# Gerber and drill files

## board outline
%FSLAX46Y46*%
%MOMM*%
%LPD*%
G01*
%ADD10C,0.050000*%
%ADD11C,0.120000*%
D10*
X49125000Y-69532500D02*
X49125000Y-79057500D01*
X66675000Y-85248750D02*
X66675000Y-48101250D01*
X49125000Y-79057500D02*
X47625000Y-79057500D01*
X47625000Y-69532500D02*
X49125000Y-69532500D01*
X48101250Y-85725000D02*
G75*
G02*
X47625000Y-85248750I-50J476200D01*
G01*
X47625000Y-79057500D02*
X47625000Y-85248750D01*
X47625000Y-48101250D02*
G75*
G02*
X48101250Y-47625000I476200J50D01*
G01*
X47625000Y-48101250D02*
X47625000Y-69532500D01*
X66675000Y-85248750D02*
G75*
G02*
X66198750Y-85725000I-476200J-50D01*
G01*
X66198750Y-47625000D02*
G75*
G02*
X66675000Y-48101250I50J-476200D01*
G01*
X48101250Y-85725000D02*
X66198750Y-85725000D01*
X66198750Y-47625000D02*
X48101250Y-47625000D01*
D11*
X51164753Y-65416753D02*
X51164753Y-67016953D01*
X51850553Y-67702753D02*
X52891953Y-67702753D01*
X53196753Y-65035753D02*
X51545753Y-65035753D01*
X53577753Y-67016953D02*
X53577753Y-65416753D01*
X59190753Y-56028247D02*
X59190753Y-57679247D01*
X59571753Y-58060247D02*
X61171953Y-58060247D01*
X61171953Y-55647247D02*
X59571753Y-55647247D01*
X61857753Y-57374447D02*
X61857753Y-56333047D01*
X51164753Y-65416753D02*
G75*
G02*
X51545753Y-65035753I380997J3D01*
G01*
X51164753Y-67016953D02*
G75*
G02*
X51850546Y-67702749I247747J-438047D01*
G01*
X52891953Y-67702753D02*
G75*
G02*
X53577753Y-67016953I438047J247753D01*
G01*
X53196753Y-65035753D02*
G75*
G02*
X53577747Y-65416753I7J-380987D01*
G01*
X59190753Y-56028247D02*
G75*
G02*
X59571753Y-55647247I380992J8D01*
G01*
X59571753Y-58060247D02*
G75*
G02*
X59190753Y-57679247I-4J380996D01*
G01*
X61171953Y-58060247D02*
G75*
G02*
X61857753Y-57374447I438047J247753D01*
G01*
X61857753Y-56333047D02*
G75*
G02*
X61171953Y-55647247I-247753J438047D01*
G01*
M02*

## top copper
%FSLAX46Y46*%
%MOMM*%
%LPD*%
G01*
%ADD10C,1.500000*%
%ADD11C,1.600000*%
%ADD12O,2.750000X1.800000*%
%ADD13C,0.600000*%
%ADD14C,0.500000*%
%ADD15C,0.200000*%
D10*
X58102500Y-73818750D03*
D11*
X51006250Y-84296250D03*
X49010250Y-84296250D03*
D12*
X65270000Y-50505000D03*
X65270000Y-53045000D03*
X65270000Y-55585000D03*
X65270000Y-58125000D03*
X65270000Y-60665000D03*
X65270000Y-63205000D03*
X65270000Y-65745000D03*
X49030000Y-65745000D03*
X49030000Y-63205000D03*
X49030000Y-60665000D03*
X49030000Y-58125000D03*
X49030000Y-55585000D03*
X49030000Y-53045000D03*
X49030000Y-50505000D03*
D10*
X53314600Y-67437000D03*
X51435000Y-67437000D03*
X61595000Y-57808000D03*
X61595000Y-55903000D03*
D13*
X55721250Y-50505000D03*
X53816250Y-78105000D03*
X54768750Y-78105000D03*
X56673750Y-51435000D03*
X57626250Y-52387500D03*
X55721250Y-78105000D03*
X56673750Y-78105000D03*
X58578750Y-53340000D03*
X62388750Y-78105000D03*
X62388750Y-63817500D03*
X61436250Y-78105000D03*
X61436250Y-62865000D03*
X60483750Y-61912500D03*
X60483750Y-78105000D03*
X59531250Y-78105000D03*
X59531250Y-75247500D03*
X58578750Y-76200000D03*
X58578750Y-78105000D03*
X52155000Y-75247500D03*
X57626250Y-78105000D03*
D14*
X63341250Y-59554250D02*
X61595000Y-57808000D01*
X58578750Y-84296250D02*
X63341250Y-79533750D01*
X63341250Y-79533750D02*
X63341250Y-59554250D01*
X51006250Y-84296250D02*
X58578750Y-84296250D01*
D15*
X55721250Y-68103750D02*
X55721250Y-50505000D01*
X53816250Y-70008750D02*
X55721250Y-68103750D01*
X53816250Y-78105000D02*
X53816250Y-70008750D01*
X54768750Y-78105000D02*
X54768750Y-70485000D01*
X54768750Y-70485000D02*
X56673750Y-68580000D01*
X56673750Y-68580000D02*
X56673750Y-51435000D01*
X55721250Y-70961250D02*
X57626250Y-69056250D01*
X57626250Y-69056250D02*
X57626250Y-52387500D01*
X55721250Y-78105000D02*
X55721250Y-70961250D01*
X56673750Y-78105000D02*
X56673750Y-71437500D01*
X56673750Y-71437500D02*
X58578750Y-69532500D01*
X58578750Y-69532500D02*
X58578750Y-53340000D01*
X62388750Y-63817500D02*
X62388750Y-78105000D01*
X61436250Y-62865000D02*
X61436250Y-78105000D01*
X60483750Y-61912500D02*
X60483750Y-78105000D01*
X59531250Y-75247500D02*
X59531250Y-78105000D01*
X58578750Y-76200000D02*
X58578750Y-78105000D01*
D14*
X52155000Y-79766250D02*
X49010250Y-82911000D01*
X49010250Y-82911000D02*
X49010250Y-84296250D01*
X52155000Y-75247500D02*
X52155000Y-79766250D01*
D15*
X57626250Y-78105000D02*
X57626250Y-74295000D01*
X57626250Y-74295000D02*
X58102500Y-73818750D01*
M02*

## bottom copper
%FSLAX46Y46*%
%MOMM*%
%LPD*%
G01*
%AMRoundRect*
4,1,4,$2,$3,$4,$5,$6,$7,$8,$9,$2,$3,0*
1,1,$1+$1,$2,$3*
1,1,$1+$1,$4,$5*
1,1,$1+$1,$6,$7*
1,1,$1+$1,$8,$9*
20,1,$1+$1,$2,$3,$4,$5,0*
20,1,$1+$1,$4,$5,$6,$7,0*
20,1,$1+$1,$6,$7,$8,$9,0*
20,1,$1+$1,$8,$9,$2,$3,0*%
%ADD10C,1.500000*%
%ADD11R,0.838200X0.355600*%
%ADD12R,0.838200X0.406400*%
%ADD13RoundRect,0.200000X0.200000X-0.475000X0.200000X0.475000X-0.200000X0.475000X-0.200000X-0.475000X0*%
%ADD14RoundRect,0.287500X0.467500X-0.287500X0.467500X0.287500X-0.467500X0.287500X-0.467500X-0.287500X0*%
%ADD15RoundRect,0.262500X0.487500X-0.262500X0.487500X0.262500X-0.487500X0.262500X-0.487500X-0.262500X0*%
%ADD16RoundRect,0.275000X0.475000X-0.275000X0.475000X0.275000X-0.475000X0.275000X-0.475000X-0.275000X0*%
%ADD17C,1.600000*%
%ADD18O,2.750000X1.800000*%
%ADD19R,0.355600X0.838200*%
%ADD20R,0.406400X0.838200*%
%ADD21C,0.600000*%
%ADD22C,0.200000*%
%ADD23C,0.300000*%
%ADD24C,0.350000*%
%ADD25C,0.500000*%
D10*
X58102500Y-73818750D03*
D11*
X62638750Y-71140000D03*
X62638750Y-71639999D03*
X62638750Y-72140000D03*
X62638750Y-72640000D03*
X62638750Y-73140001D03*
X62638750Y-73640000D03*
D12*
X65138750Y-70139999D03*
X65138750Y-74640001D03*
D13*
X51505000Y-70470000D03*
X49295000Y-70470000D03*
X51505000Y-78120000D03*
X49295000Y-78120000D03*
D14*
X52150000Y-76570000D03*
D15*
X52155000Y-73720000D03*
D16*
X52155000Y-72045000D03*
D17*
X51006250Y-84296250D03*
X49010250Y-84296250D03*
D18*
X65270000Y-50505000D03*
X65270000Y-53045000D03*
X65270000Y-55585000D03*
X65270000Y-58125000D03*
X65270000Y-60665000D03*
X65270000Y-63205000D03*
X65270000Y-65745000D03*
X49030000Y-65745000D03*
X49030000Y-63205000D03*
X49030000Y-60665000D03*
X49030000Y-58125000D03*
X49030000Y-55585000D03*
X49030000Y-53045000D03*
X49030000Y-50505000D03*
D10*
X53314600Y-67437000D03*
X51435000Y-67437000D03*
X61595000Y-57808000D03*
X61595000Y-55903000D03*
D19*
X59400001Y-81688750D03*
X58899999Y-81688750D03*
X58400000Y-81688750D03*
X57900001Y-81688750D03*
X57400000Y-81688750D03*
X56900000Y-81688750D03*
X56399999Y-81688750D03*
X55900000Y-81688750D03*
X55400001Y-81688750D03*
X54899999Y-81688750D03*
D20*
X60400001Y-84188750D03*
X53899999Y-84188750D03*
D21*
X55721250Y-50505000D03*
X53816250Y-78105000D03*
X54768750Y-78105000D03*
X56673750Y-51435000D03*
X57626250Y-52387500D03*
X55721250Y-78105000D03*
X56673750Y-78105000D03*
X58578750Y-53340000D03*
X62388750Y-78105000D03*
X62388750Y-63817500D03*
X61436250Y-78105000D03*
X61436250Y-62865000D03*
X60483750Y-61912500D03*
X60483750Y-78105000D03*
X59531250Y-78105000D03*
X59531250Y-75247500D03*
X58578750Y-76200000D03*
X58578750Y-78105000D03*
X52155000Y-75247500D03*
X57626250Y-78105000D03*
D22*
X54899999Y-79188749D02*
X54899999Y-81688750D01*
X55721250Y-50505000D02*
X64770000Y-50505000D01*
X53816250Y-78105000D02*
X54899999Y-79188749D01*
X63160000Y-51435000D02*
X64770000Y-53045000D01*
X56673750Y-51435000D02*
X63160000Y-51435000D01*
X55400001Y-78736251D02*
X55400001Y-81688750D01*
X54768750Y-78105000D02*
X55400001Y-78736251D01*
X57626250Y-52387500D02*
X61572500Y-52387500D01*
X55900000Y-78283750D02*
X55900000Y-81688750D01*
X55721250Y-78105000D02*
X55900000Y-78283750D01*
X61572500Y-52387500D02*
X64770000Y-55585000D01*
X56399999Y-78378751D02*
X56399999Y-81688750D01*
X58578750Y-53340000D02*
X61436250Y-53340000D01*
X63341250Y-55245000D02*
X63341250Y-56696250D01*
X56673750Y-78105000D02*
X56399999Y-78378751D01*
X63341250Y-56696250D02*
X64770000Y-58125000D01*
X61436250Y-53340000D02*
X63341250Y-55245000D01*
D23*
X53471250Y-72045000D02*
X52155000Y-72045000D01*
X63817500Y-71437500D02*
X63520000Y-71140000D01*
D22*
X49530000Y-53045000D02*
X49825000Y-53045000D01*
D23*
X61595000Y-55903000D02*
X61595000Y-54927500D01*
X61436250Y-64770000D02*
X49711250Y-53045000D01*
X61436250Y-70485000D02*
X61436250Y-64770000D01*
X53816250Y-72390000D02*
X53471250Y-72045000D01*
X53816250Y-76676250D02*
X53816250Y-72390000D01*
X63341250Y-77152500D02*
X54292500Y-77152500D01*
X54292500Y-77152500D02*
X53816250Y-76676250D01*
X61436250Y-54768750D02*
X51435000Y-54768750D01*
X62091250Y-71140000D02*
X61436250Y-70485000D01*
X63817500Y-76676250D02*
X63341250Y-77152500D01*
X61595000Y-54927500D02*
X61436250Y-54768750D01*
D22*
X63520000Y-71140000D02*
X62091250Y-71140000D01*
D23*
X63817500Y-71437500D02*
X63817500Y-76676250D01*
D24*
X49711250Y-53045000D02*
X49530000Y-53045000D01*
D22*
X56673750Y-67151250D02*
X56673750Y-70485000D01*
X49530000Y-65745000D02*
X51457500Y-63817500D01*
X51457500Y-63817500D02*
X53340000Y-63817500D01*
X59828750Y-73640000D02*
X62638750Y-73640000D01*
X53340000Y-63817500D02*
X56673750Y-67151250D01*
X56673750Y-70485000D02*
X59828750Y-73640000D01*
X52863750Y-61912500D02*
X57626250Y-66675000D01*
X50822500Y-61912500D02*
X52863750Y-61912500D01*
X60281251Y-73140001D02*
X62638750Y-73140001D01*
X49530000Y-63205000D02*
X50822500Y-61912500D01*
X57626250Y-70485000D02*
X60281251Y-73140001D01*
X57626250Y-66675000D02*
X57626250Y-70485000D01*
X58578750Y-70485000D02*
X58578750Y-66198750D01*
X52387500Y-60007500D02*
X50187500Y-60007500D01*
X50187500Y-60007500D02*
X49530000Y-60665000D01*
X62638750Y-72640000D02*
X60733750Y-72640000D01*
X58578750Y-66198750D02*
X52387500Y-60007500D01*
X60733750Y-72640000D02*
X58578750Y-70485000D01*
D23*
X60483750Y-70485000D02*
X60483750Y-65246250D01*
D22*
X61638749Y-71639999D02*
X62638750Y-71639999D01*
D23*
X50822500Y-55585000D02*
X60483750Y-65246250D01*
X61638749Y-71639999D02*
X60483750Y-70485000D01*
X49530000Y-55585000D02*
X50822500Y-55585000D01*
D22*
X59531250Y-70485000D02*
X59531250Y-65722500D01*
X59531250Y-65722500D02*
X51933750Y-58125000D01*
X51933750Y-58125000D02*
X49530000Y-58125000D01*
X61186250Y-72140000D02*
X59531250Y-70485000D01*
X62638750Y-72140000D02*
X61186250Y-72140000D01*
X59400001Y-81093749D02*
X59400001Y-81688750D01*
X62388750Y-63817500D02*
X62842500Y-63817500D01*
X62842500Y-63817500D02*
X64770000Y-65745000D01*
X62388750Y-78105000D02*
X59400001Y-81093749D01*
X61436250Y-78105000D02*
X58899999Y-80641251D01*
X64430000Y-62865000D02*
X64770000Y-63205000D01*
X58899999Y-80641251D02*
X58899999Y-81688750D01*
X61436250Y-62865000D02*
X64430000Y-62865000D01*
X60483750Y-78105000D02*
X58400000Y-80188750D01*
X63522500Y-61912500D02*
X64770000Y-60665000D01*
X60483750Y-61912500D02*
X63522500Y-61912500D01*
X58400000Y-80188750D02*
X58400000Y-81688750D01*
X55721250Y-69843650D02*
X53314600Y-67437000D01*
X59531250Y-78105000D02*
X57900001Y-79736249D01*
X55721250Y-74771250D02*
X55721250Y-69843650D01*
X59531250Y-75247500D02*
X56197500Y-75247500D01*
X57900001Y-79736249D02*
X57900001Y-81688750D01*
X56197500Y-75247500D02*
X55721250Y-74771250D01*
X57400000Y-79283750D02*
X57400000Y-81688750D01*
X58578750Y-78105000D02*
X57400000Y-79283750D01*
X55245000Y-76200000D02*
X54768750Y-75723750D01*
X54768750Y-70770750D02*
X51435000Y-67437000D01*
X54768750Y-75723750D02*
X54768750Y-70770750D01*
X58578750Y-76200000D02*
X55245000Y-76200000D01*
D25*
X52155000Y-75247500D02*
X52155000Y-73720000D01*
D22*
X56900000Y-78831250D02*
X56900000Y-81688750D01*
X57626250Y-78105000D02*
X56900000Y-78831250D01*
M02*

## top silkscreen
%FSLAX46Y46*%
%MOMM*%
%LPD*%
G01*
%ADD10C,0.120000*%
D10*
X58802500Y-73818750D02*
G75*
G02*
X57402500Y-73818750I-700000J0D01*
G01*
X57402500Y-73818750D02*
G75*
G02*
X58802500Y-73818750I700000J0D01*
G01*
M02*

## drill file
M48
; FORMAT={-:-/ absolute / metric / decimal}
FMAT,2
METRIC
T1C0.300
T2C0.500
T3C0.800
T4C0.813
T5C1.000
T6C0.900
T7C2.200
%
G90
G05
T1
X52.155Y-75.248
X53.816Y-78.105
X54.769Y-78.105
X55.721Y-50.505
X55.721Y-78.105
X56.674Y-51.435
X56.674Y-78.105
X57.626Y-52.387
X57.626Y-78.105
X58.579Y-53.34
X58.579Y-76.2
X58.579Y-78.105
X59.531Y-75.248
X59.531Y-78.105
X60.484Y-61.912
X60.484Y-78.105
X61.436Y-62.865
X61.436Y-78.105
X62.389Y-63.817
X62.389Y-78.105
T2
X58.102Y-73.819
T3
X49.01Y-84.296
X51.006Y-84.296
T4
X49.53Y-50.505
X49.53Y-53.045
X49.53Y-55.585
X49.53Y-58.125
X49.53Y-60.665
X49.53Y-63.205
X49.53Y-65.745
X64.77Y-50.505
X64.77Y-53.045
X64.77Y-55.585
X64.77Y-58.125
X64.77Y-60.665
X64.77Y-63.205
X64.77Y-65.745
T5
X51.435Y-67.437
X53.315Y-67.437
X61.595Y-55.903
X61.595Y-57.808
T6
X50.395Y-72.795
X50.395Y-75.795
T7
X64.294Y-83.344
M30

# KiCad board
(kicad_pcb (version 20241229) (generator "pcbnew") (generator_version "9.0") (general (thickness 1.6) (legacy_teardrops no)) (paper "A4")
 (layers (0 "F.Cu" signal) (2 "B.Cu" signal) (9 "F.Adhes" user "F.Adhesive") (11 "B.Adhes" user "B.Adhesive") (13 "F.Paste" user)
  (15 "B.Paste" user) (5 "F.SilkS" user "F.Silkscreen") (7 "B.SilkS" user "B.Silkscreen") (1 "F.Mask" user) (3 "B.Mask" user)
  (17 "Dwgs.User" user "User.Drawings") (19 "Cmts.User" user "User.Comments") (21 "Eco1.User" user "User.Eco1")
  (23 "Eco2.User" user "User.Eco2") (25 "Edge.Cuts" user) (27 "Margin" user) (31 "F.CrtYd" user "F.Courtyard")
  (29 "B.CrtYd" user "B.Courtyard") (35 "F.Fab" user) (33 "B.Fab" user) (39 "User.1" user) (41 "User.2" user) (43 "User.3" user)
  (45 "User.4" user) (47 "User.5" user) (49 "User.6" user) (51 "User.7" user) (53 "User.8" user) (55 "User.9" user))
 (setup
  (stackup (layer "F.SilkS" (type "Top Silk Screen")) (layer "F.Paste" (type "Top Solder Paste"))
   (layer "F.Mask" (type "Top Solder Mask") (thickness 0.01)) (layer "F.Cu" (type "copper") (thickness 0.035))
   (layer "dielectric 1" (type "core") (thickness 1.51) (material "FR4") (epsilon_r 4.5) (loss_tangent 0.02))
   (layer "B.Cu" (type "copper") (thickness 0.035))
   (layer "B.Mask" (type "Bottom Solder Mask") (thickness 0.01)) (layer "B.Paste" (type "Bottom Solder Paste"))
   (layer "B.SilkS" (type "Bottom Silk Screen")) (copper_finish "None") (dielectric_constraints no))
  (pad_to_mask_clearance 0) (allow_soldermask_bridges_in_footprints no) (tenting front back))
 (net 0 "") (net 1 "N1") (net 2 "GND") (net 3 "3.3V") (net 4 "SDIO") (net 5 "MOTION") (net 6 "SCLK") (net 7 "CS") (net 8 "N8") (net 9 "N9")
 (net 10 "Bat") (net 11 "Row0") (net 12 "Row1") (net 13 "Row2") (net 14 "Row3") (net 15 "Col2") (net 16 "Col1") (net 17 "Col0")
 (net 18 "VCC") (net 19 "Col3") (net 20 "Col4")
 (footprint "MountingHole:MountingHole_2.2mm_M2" (layer "F.Cu") (at 64.29375 83.34375)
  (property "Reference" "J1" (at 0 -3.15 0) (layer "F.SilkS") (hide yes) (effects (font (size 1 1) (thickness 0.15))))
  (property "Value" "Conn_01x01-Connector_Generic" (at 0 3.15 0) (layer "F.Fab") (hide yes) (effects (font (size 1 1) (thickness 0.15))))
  (pad "" np_thru_hole circle (at 0 0) (size 2.2 2.2) (drill 2.2) (layers "*.Cu" "*.Mask")))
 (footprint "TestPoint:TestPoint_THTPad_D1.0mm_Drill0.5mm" (layer "F.Cu") (at 58.1025 73.81875)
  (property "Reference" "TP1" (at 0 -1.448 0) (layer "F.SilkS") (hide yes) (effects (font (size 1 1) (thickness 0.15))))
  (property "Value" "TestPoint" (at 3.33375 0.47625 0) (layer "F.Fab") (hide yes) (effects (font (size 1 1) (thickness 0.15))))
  (fp_circle (center 0 0) (end 0 0.7) (stroke (width 0.12) (type solid)) (fill no) (layer "F.SilkS"))
  (pad "1" thru_hole circle (at 0 0) (size 1.5 1.5) (drill 0.5) (layers "*.Cu" "*.Mask") (remove_unused_layers no) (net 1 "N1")))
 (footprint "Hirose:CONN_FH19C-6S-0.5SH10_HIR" (layer "B.Cu") (at 64.29375 72.39 -90)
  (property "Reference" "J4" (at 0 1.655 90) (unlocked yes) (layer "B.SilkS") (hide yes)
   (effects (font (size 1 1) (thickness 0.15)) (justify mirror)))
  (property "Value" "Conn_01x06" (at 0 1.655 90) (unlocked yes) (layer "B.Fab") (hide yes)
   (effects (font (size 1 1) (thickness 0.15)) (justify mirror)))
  (pad "1" smd rect (at -1.25 1.655 270) (size 0.3556 0.8382) (layers "B.Cu" "B.Mask" "B.Paste") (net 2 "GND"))
  (pad "2" smd rect (at -0.750001 1.655 270) (size 0.3556 0.8382) (layers "B.Cu" "B.Mask" "B.Paste") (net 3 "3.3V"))
  (pad "3" smd rect (at -0.25 1.655 270) (size 0.3556 0.8382) (layers "B.Cu" "B.Mask" "B.Paste") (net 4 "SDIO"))
  (pad "4" smd rect (at 0.25 1.655 270) (size 0.3556 0.8382) (layers "B.Cu" "B.Mask" "B.Paste") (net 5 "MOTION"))
  (pad "5" smd rect (at 0.750001 1.655 270) (size 0.3556 0.8382) (layers "B.Cu" "B.Mask" "B.Paste") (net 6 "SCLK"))
  (pad "6" smd rect (at 1.25 1.655 270) (size 0.3556 0.8382) (layers "B.Cu" "B.Mask" "B.Paste") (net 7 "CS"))
  (pad "7" smd rect (at -2.250001 -0.845 270) (size 0.4064 0.8382) (layers "B.Cu" "B.Mask" "B.Paste"))
  (pad "8" smd rect (at 2.250001 -0.845 270) (size 0.4064 0.8382) (layers "B.Cu" "B.Mask" "B.Paste")))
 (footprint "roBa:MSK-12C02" (layer "B.Cu") (at 50.395 74.295 -90)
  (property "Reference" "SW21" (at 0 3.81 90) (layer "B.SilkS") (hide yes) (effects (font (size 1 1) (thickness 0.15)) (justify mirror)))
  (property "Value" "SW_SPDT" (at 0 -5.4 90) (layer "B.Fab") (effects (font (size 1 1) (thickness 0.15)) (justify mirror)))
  (pad "" smd roundrect (at -3.825 -1.11 90) (size 1.35 0.8) (layers "B.Cu" "B.Mask" "B.Paste") (roundrect_rratio 0.25))
  (pad "" smd roundrect (at -3.825 1.1 90) (size 1.35 0.8) (layers "B.Cu" "B.Mask" "B.Paste") (roundrect_rratio 0.25))
  (pad "" np_thru_hole circle (at -1.5 0 90) (size 0.9 0.9) (drill 0.9) (layers "*.Cu" "*.Mask"))
  (pad "" np_thru_hole circle (at 1.5 0 90) (size 0.9 0.9) (drill 0.9) (layers "*.Cu" "*.Mask"))
  (pad "" smd roundrect (at 3.825 -1.11 90) (size 1.35 0.8) (layers "B.Cu" "B.Mask" "B.Paste") (roundrect_rratio 0.25))
  (pad "" smd roundrect (at 3.825 1.1 90) (size 1.35 0.8) (layers "B.Cu" "B.Mask" "B.Paste") (roundrect_rratio 0.25))
  (pad "1" smd roundrect (at 2.275 -1.755 90) (size 1.15 1.51) (layers "B.Cu" "B.Mask" "B.Paste") (roundrect_rratio 0.25) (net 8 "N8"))
  (pad "2" smd roundrect (at -0.575 -1.76 90) (size 1.05 1.5) (layers "B.Cu" "B.Mask" "B.Paste") (roundrect_rratio 0.25) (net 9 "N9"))
  (pad "3" smd roundrect (at -2.25 -1.76 90) (size 1.1 1.5) (layers "B.Cu" "B.Mask" "B.Paste") (roundrect_rratio 0.25) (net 2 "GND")))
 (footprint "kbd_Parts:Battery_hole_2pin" (layer "B.Cu") (at 50.00625 84.29625 90)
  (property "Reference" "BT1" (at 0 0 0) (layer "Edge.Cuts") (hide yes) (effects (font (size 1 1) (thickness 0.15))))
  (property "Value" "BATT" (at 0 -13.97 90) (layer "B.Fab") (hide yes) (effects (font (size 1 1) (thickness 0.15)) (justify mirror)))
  (pad "1" thru_hole circle (at 0 1 90) (size 1.6 1.6) (drill 0.8) (layers "*.Cu" "*.Mask" "B.SilkS") (remove_unused_layers no)
   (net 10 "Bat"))
  (pad "2" thru_hole circle (at 0 -0.996 90) (size 1.6 1.6) (drill 0.8) (layers "*.Cu" "*.Mask" "B.SilkS") (remove_unused_layers no)
   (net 9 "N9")))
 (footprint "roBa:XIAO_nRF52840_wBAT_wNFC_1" (layer "B.Cu") (at 57.15 47.625 180)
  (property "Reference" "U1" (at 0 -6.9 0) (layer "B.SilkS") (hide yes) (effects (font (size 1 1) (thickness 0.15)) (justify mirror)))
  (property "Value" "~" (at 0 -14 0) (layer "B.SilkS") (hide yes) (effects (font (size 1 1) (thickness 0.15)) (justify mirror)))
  (fp_line (start 5.985247 -17.791753) (end 5.985247 -19.391953) (stroke (width 0.12) (type solid)) (layer "Edge.Cuts"))
  (fp_line (start 5.299447 -20.077753) (end 4.258047 -20.077753) (stroke (width 0.12) (type solid)) (layer "Edge.Cuts"))
  (fp_line (start 3.953247 -17.410753) (end 5.604247 -17.410753) (stroke (width 0.12) (type solid)) (layer "Edge.Cuts"))
  (fp_line (start 3.572247 -19.391953) (end 3.572247 -17.791753) (stroke (width 0.12) (type solid)) (layer "Edge.Cuts"))
  (fp_line (start -2.040753 -8.403247) (end -2.040753 -10.054247) (stroke (width 0.12) (type solid)) (layer "Edge.Cuts"))
  (fp_line (start -2.421753 -10.435247) (end -4.021953 -10.435247) (stroke (width 0.12) (type solid)) (layer "Edge.Cuts"))
  (fp_line (start -4.021953 -8.022247) (end -2.421753 -8.022247) (stroke (width 0.12) (type solid)) (layer "Edge.Cuts"))
  (fp_line (start -4.707753 -9.749447) (end -4.707753 -8.708047) (stroke (width 0.12) (type solid)) (layer "Edge.Cuts"))
  (fp_arc (start 5.985247 -17.791753) (mid 5.873656 -17.522344) (end 5.604247 -17.410753) (stroke (width 0.12) (type solid))
   (layer "Edge.Cuts"))
  (fp_arc (start 5.985247 -19.391953) (mid 5.381645 -19.474147) (end 5.299447 -20.077753) (stroke (width 0.12) (type solid))
   (layer "Edge.Cuts"))
  (fp_arc (start 4.258047 -20.077753) (mid 4.175856 -19.474144) (end 3.572247 -19.391953) (stroke (width 0.12) (type solid))
   (layer "Edge.Cuts"))
  (fp_arc (start 3.953247 -17.410753) (mid 3.683836 -17.522343) (end 3.572247 -17.791753) (stroke (width 0.12) (type solid))
   (layer "Edge.Cuts"))
  (fp_arc (start -2.040753 -8.403247) (mid -2.152343 -8.133837) (end -2.421753 -8.022247) (stroke (width 0.12) (type solid))
   (layer "Edge.Cuts"))
  (fp_arc (start -2.421753 -10.435247) (mid -2.152344 -10.323656) (end -2.040753 -10.054247) (stroke (width 0.12) (type solid))
   (layer "Edge.Cuts"))
  (fp_arc (start -4.021953 -10.435247) (mid -4.104144 -9.831638) (end -4.707753 -9.749447) (stroke (width 0.12) (type solid))
   (layer "Edge.Cuts"))
  (fp_arc (start -4.707753 -8.708047) (mid -4.104144 -8.625856) (end -4.021953 -8.022247) (stroke (width 0.12) (type solid))
   (layer "Edge.Cuts"))
  (pad "1" thru_hole oval (at -7.62 -2.88 180) (size 2.75 1.8) (drill 0.8128 (offset -0.5 0)) (layers "*.Cu" "*.Mask")
   (remove_unused_layers no) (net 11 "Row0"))
  (pad "2" thru_hole oval (at -7.62 -5.42 180) (size 2.75 1.8) (drill 0.8128 (offset -0.5 0)) (layers "*.Cu" "*.Mask")
   (remove_unused_layers no) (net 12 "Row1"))
  (pad "3" thru_hole oval (at -7.62 -7.96 180) (size 2.75 1.8) (drill 0.8128 (offset -0.5 0)) (layers "*.Cu" "*.Mask")
   (remove_unused_layers no) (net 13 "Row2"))
  (pad "4" thru_hole oval (at -7.62 -10.5 180) (size 2.75 1.8) (drill 0.8128 (offset -0.5 0)) (layers "*.Cu" "*.Mask")
   (remove_unused_layers no) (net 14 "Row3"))
  (pad "5" thru_hole oval (at -7.62 -13.04 180) (size 2.75 1.8) (drill 0.8128 (offset -0.5 0)) (layers "*.Cu" "*.Mask")
   (remove_unused_layers no) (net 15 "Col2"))
  (pad "6" thru_hole oval (at -7.62 -15.58 180) (size 2.75 1.8) (drill 0.8128 (offset -0.5 0)) (layers "*.Cu" "*.Mask")
   (remove_unused_layers no) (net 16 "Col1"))
  (pad "7" thru_hole oval (at -7.62 -18.12 180) (size 2.75 1.8) (drill 0.8128 (offset -0.5 0)) (layers "*.Cu" "*.Mask")
   (remove_unused_layers no) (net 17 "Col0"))
  (pad "8" thru_hole oval (at 7.62 -18.12 180) (size 2.75 1.8) (drill 0.8128 (offset 0.5 0)) (layers "*.Cu" "*.Mask")
   (remove_unused_layers no) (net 7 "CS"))
  (pad "9" thru_hole oval (at 7.62 -15.58 180) (size 2.75 1.8) (drill 0.8128 (offset 0.5 0)) (layers "*.Cu" "*.Mask")
   (remove_unused_layers no) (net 6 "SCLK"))
  (pad "10" thru_hole oval (at 7.62 -13.04 180) (size 2.75 1.8) (drill 0.8128 (offset 0.5 0)) (layers "*.Cu" "*.Mask")
   (remove_unused_layers no) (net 5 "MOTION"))
  (pad "11" thru_hole oval (at 7.62 -10.5 180) (size 2.75 1.8) (drill 0.8128 (offset 0.5 0)) (layers "*.Cu" "*.Mask")
   (remove_unused_layers no) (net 4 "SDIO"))
  (pad "12" thru_hole oval (at 7.62 -7.96 180) (size 2.75 1.8) (drill 0.8128 (offset 0.5 0)) (layers "*.Cu" "*.Mask")
   (remove_unused_layers no) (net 3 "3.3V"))
  (pad "13" thru_hole oval (at 7.62 -5.42 180) (size 2.75 1.8) (drill 0.8128 (offset 0.5 0)) (layers "*.Cu" "*.Mask")
   (remove_unused_layers no) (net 2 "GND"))
  (pad "14" thru_hole oval (at 7.62 -2.88 180) (size 2.75 1.8) (drill 0.8128 (offset 0.5 0)) (layers "*.Cu" "*.Mask")
   (remove_unused_layers no) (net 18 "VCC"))
  (pad "15" thru_hole circle (at 3.8354 -19.812 90) (size 1.5 1.5) (drill 1) (layers "*.Cu" "*.Mask") (remove_unused_layers no)
   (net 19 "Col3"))
  (pad "16" thru_hole circle (at 5.715 -19.812 270) (size 1.5 1.5) (drill 1) (layers "*.Cu" "*.Mask") (remove_unused_layers no)
   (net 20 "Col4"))
  (pad "20" thru_hole circle (at -4.445 -10.183 270) (size 1.5 1.5) (drill 1) (layers "*.Cu" "*.Mask") (remove_unused_layers no)
   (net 10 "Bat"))
  (pad "21" thru_hole circle (at -4.445 -8.278 90) (size 1.5 1.5) (drill 1) (layers "*.Cu" "*.Mask") (remove_unused_layers no) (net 2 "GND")))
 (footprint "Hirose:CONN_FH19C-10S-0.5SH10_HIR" (layer "B.Cu") (at 57.15 83.34375 180)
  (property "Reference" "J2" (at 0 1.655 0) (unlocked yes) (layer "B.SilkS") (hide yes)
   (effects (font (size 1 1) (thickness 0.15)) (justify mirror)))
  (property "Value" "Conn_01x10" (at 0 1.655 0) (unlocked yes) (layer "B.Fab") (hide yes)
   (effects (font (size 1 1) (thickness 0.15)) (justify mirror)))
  (pad "1" smd rect (at -2.250001 1.655 180) (size 0.3556 0.8382) (layers "B.Cu" "B.Mask" "B.Paste") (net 17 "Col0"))
  (pad "2" smd rect (at -1.749999 1.655 180) (size 0.3556 0.8382) (layers "B.Cu" "B.Mask" "B.Paste") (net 16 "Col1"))
  (pad "3" smd rect (at -1.25 1.655 180) (size 0.3556 0.8382) (layers "B.Cu" "B.Mask" "B.Paste") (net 15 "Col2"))
  (pad "4" smd rect (at -0.750001 1.655 180) (size 0.3556 0.8382) (layers "B.Cu" "B.Mask" "B.Paste") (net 19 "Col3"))
  (pad "5" smd rect (at -0.25 1.655 180) (size 0.3556 0.8382) (layers "B.Cu" "B.Mask" "B.Paste") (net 20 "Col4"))
  (pad "6" smd rect (at 0.25 1.655 180) (size 0.3556 0.8382) (layers "B.Cu" "B.Mask" "B.Paste") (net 1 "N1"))
  (pad "7" smd rect (at 0.750001 1.655 180) (size 0.3556 0.8382) (layers "B.Cu" "B.Mask" "B.Paste") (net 14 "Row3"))
  (pad "8" smd rect (at 1.25 1.655 180) (size 0.3556 0.8382) (layers "B.Cu" "B.Mask" "B.Paste") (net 13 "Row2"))
  (pad "9" smd rect (at 1.749999 1.655 180) (size 0.3556 0.8382) (layers "B.Cu" "B.Mask" "B.Paste") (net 12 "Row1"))
  (pad "10" smd rect (at 2.250001 1.655 180) (size 0.3556 0.8382) (layers "B.Cu" "B.Mask" "B.Paste") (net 11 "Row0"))
  (pad "11" smd rect (at -3.250001 -0.845 180) (size 0.4064 0.8382) (layers "B.Cu" "B.Mask" "B.Paste"))
  (pad "12" smd rect (at 3.250001 -0.845 180) (size 0.4064 0.8382) (layers "B.Cu" "B.Mask" "B.Paste")))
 (gr_line (start 49.125 69.5325) (end 49.125 79.0575) (stroke (width 0.05) (type solid)) (layer "Edge.Cuts"))
 (gr_line (start 66.675 85.24875) (end 66.675 48.10125) (stroke (width 0.05) (type default)) (layer "Edge.Cuts"))
 (gr_line (start 49.125 79.0575) (end 47.625 79.0575) (stroke (width 0.05) (type default)) (layer "Edge.Cuts"))
 (gr_line (start 47.625 69.5325) (end 49.125 69.5325) (stroke (width 0.05) (type default)) (layer "Edge.Cuts"))
 (gr_arc (start 48.10125 85.725) (mid 47.76449 85.58551) (end 47.625 85.24875) (stroke (width 0.05) (type default)) (layer "Edge.Cuts"))
 (gr_line (start 47.625 79.0575) (end 47.625 85.24875) (stroke (width 0.05) (type default)) (layer "Edge.Cuts"))
 (gr_arc (start 47.625 48.10125) (mid 47.76449 47.76449) (end 48.10125 47.625) (stroke (width 0.05) (type default)) (layer "Edge.Cuts"))
 (gr_line (start 47.625 48.10125) (end 47.625 69.5325) (stroke (width 0.05) (type default)) (layer "Edge.Cuts"))
 (gr_arc (start 66.675 85.24875) (mid 66.53551 85.58551) (end 66.19875 85.725) (stroke (width 0.05) (type default)) (layer "Edge.Cuts"))
 (gr_arc (start 66.19875 47.625) (mid 66.53551 47.76449) (end 66.675 48.10125) (stroke (width 0.05) (type default)) (layer "Edge.Cuts"))
 (gr_line (start 48.10125 85.725) (end 66.19875 85.725) (stroke (width 0.05) (type default)) (layer "Edge.Cuts"))
 (gr_line (start 66.19875 47.625) (end 48.10125 47.625) (stroke (width 0.05) (type default)) (layer "Edge.Cuts"))
 (segment (start 63.34125 59.55425) (end 61.595 57.808) (width 0.5) (layer "F.Cu") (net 10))
 (segment (start 58.57875 84.29625) (end 63.34125 79.53375) (width 0.5) (layer "F.Cu") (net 10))
 (segment (start 63.34125 79.53375) (end 63.34125 59.55425) (width 0.5) (layer "F.Cu") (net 10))
 (segment (start 51.00625 84.29625) (end 58.57875 84.29625) (width 0.5) (layer "F.Cu") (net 10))
 (segment (start 55.72125 68.10375) (end 55.72125 50.505) (width 0.2) (layer "F.Cu") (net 11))
 (segment (start 53.81625 70.00875) (end 55.72125 68.10375) (width 0.2) (layer "F.Cu") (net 11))
 (segment (start 53.81625 78.105) (end 53.81625 70.00875) (width 0.2) (layer "F.Cu") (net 11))
 (via (at 55.72125 50.505) (size 0.6) (drill 0.3) (layers "F.Cu" "B.Cu") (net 11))
 (via (at 53.81625 78.105) (size 0.6) (drill 0.3) (layers "F.Cu" "B.Cu") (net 11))
 (segment (start 54.899999 79.188749) (end 54.899999 81.68875) (width 0.2) (layer "B.Cu") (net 11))
 (segment (start 55.72125 50.505) (end 64.77 50.505) (width 0.2) (layer "B.Cu") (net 11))
 (segment (start 53.81625 78.105) (end 54.899999 79.188749) (width 0.2) (layer "B.Cu") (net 11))
 (segment (start 54.76875 78.105) (end 54.76875 70.485) (width 0.2) (layer "F.Cu") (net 12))
 (segment (start 54.76875 70.485) (end 56.67375 68.58) (width 0.2) (layer "F.Cu") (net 12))
 (segment (start 56.67375 68.58) (end 56.67375 51.435) (width 0.2) (layer "F.Cu") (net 12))
 (via (at 54.76875 78.105) (size 0.6) (drill 0.3) (layers "F.Cu" "B.Cu") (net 12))
 (via (at 56.67375 51.435) (size 0.6) (drill 0.3) (layers "F.Cu" "B.Cu") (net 12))
 (segment (start 63.16 51.435) (end 64.77 53.045) (width 0.2) (layer "B.Cu") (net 12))
 (segment (start 56.67375 51.435) (end 63.16 51.435) (width 0.2) (layer "B.Cu") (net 12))
 (segment (start 55.400001 78.736251) (end 55.400001 81.68875) (width 0.2) (layer "B.Cu") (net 12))
 (segment (start 54.76875 78.105) (end 55.400001 78.736251) (width 0.2) (layer "B.Cu") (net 12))
 (segment (start 55.72125 70.96125) (end 57.62625 69.05625) (width 0.2) (layer "F.Cu") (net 13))
 (segment (start 57.62625 69.05625) (end 57.62625 52.3875) (width 0.2) (layer "F.Cu") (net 13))
 (segment (start 55.72125 78.105) (end 55.72125 70.96125) (width 0.2) (layer "F.Cu") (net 13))
 (via (at 57.62625 52.3875) (size 0.6) (drill 0.3) (layers "F.Cu" "B.Cu") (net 13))
 (via (at 55.72125 78.105) (size 0.6) (drill 0.3) (layers "F.Cu" "B.Cu") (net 13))
 (segment (start 57.62625 52.3875) (end 61.5725 52.3875) (width 0.2) (layer "B.Cu") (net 13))
 (segment (start 55.9 78.28375) (end 55.9 81.68875) (width 0.2) (layer "B.Cu") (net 13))
 (segment (start 55.72125 78.105) (end 55.9 78.28375) (width 0.2) (layer "B.Cu") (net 13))
 (segment (start 61.5725 52.3875) (end 64.77 55.585) (width 0.2) (layer "B.Cu") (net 13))
 (segment (start 56.67375 78.105) (end 56.67375 71.4375) (width 0.2) (layer "F.Cu") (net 14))
 (segment (start 56.67375 71.4375) (end 58.57875 69.5325) (width 0.2) (layer "F.Cu") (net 14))
 (segment (start 58.57875 69.5325) (end 58.57875 53.34) (width 0.2) (layer "F.Cu") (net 14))
 (via (at 56.67375 78.105) (size 0.6) (drill 0.3) (layers "F.Cu" "B.Cu") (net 14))
 (via (at 58.57875 53.34) (size 0.6) (drill 0.3) (layers "F.Cu" "B.Cu") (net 14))
 (segment (start 56.399999 78.378751) (end 56.399999 81.68875) (width 0.2) (layer "B.Cu") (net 14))
 (segment (start 58.57875 53.34) (end 61.43625 53.34) (width 0.2) (layer "B.Cu") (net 14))
 (segment (start 63.34125 55.245) (end 63.34125 56.69625) (width 0.2) (layer "B.Cu") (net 14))
 (segment (start 56.67375 78.105) (end 56.399999 78.378751) (width 0.2) (layer "B.Cu") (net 14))
 (segment (start 63.34125 56.69625) (end 64.77 58.125) (width 0.2) (layer "B.Cu") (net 14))
 (segment (start 61.43625 53.34) (end 63.34125 55.245) (width 0.2) (layer "B.Cu") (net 14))
 (segment (start 53.47125 72.045) (end 52.155 72.045) (width 0.3) (layer "B.Cu") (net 2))
 (segment (start 63.8175 71.4375) (end 63.52 71.14) (width 0.3) (layer "B.Cu") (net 2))
 (segment (start 49.53 53.045) (end 49.825 53.045) (width 0.2) (layer "B.Cu") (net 2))
 (segment (start 61.595 55.903) (end 61.595 54.9275) (width 0.3) (layer "B.Cu") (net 2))
 (segment (start 61.43625 64.77) (end 49.71125 53.045) (width 0.3) (layer "B.Cu") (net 2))
 (segment (start 61.43625 70.485) (end 61.43625 64.77) (width 0.3) (layer "B.Cu") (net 2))
 (segment (start 53.81625 72.39) (end 53.47125 72.045) (width 0.3) (layer "B.Cu") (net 2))
 (segment (start 53.81625 76.67625) (end 53.81625 72.39) (width 0.3) (layer "B.Cu") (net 2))
 (segment (start 63.34125 77.1525) (end 54.2925 77.1525) (width 0.3) (layer "B.Cu") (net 2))
 (segment (start 54.2925 77.1525) (end 53.81625 76.67625) (width 0.3) (layer "B.Cu") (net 2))
 (segment (start 61.43625 54.76875) (end 51.435 54.76875) (width 0.3) (layer "B.Cu") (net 2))
 (segment (start 62.09125 71.14) (end 61.43625 70.485) (width 0.3) (layer "B.Cu") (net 2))
 (segment (start 63.8175 76.67625) (end 63.34125 77.1525) (width 0.3) (layer "B.Cu") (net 2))
 (segment (start 61.595 54.9275) (end 61.43625 54.76875) (width 0.3) (layer "B.Cu") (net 2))
 (segment (start 63.52 71.14) (end 62.09125 71.14) (width 0.2) (layer "B.Cu") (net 2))
 (segment (start 63.8175 71.4375) (end 63.8175 76.67625) (width 0.3) (layer "B.Cu") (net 2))
 (segment (start 49.71125 53.045) (end 49.53 53.045) (width 0.35) (layer "B.Cu") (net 2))
 (segment (start 56.67375 67.15125) (end 56.67375 70.485) (width 0.2) (layer "B.Cu") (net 7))
 (segment (start 49.53 65.745) (end 51.4575 63.8175) (width 0.2) (layer "B.Cu") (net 7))
 (segment (start 51.4575 63.8175) (end 53.34 63.8175) (width 0.2) (layer "B.Cu") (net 7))
 (segment (start 59.82875 73.64) (end 62.63875 73.64) (width 0.2) (layer "B.Cu") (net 7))
 (segment (start 53.34 63.8175) (end 56.67375 67.15125) (width 0.2) (layer "B.Cu") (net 7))
 (segment (start 56.67375 70.485) (end 59.82875 73.64) (width 0.2) (layer "B.Cu") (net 7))
 (segment (start 52.86375 61.9125) (end 57.62625 66.675) (width 0.2) (layer "B.Cu") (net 6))
 (segment (start 50.8225 61.9125) (end 52.86375 61.9125) (width 0.2) (layer "B.Cu") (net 6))
 (segment (start 60.281251 73.140001) (end 62.63875 73.140001) (width 0.2) (layer "B.Cu") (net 6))
 (segment (start 49.53 63.205) (end 50.8225 61.9125) (width 0.2) (layer "B.Cu") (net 6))
 (segment (start 57.62625 70.485) (end 60.281251 73.140001) (width 0.2) (layer "B.Cu") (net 6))
 (segment (start 57.62625 66.675) (end 57.62625 70.485) (width 0.2) (layer "B.Cu") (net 6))
 (segment (start 58.57875 70.485) (end 58.57875 66.19875) (width 0.2) (layer "B.Cu") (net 5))
 (segment (start 52.3875 60.0075) (end 50.1875 60.0075) (width 0.2) (layer "B.Cu") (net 5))
 (segment (start 50.1875 60.0075) (end 49.53 60.665) (width 0.2) (layer "B.Cu") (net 5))
 (segment (start 62.63875 72.64) (end 60.73375 72.64) (width 0.2) (layer "B.Cu") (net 5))
 (segment (start 58.57875 66.19875) (end 52.3875 60.0075) (width 0.2) (layer "B.Cu") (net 5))
 (segment (start 60.73375 72.64) (end 58.57875 70.485) (width 0.2) (layer "B.Cu") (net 5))
 (segment (start 60.48375 70.485) (end 60.48375 65.24625) (width 0.3) (layer "B.Cu") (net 3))
 (segment (start 61.638749 71.639999) (end 62.63875 71.639999) (width 0.2) (layer "B.Cu") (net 3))
 (segment (start 50.8225 55.585) (end 60.48375 65.24625) (width 0.3) (layer "B.Cu") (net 3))
 (segment (start 61.638749 71.639999) (end 60.48375 70.485) (width 0.3) (layer "B.Cu") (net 3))
 (segment (start 49.53 55.585) (end 50.8225 55.585) (width 0.3) (layer "B.Cu") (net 3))
 (segment (start 59.53125 70.485) (end 59.53125 65.7225) (width 0.2) (layer "B.Cu") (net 4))
 (segment (start 59.53125 65.7225) (end 51.93375 58.125) (width 0.2) (layer "B.Cu") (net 4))
 (segment (start 51.93375 58.125) (end 49.53 58.125) (width 0.2) (layer "B.Cu") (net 4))
 (segment (start 61.18625 72.14) (end 59.53125 70.485) (width 0.2) (layer "B.Cu") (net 4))
 (segment (start 62.63875 72.14) (end 61.18625 72.14) (width 0.2) (layer "B.Cu") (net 4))
 (segment (start 62.38875 63.8175) (end 62.38875 78.105) (width 0.2) (layer "F.Cu") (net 17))
 (via (at 62.38875 78.105) (size 0.6) (drill 0.3) (layers "F.Cu" "B.Cu") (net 17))
 (via (at 62.38875 63.8175) (size 0.6) (drill 0.3) (layers "F.Cu" "B.Cu") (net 17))
 (segment (start 59.400001 81.093749) (end 59.400001 81.68875) (width 0.2) (layer "B.Cu") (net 17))
 (segment (start 62.38875 63.8175) (end 62.8425 63.8175) (width 0.2) (layer "B.Cu") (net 17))
 (segment (start 62.8425 63.8175) (end 64.77 65.745) (width 0.2) (layer "B.Cu") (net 17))
 (segment (start 62.38875 78.105) (end 59.400001 81.093749) (width 0.2) (layer "B.Cu") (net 17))
 (segment (start 61.43625 62.865) (end 61.43625 78.105) (width 0.2) (layer "F.Cu") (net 16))
 (via (at 61.43625 78.105) (size 0.6) (drill 0.3) (layers "F.Cu" "B.Cu") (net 16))
 (via (at 61.43625 62.865) (size 0.6) (drill 0.3) (layers "F.Cu" "B.Cu") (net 16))
 (segment (start 61.43625 78.105) (end 58.899999 80.641251) (width 0.2) (layer "B.Cu") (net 16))
 (segment (start 64.43 62.865) (end 64.77 63.205) (width 0.2) (layer "B.Cu") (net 16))
 (segment (start 58.899999 80.641251) (end 58.899999 81.68875) (width 0.2) (layer "B.Cu") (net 16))
 (segment (start 61.43625 62.865) (end 64.43 62.865) (width 0.2) (layer "B.Cu") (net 16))
 (segment (start 60.48375 61.9125) (end 60.48375 78.105) (width 0.2) (layer "F.Cu") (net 15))
 (via (at 60.48375 61.9125) (size 0.6) (drill 0.3) (layers "F.Cu" "B.Cu") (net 15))
 (via (at 60.48375 78.105) (size 0.6) (drill 0.3) (layers "F.Cu" "B.Cu") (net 15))
 (segment (start 60.48375 78.105) (end 58.4 80.18875) (width 0.2) (layer "B.Cu") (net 15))
 (segment (start 63.5225 61.9125) (end 64.77 60.665) (width 0.2) (layer "B.Cu") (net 15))
 (segment (start 60.48375 61.9125) (end 63.5225 61.9125) (width 0.2) (layer "B.Cu") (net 15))
 (segment (start 58.4 80.18875) (end 58.4 81.68875) (width 0.2) (layer "B.Cu") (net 15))
 (segment (start 59.53125 75.2475) (end 59.53125 78.105) (width 0.2) (layer "F.Cu") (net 19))
 (via (at 59.53125 78.105) (size 0.6) (drill 0.3) (layers "F.Cu" "B.Cu") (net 19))
 (via (at 59.53125 75.2475) (size 0.6) (drill 0.3) (layers "F.Cu" "B.Cu") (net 19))
 (segment (start 55.72125 69.84365) (end 53.3146 67.437) (width 0.2) (layer "B.Cu") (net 19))
 (segment (start 59.53125 78.105) (end 57.900001 79.736249) (width 0.2) (layer "B.Cu") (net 19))
 (segment (start 55.72125 74.77125) (end 55.72125 69.84365) (width 0.2) (layer "B.Cu") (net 19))
 (segment (start 59.53125 75.2475) (end 56.1975 75.2475) (width 0.2) (layer "B.Cu") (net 19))
 (segment (start 57.900001 79.736249) (end 57.900001 81.68875) (width 0.2) (layer "B.Cu") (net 19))
 (segment (start 56.1975 75.2475) (end 55.72125 74.77125) (width 0.2) (layer "B.Cu") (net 19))
 (segment (start 58.57875 76.2) (end 58.57875 78.105) (width 0.2) (layer "F.Cu") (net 20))
 (via (at 58.57875 76.2) (size 0.6) (drill 0.3) (layers "F.Cu" "B.Cu") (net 20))
 (via (at 58.57875 78.105) (size 0.6) (drill 0.3) (layers "F.Cu" "B.Cu") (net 20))
 (segment (start 57.4 79.28375) (end 57.4 81.68875) (width 0.2) (layer "B.Cu") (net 20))
 (segment (start 58.57875 78.105) (end 57.4 79.28375) (width 0.2) (layer "B.Cu") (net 20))
 (segment (start 55.245 76.2) (end 54.76875 75.72375) (width 0.2) (layer "B.Cu") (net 20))
 (segment (start 54.76875 70.77075) (end 51.435 67.437) (width 0.2) (layer "B.Cu") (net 20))
 (segment (start 54.76875 75.72375) (end 54.76875 70.77075) (width 0.2) (layer "B.Cu") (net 20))
 (segment (start 58.57875 76.2) (end 55.245 76.2) (width 0.2) (layer "B.Cu") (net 20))
 (segment (start 52.155 79.76625) (end 49.01025 82.911) (width 0.5) (layer "F.Cu") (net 9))
 (segment (start 49.01025 82.911) (end 49.01025 84.29625) (width 0.5) (layer "F.Cu") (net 9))
 (segment (start 52.155 75.2475) (end 52.155 79.76625) (width 0.5) (layer "F.Cu") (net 9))
 (via (at 52.155 75.2475) (size 0.6) (drill 0.3) (layers "F.Cu" "B.Cu") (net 9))
 (segment (start 52.155 75.2475) (end 52.155 73.72) (width 0.5) (layer "B.Cu") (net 9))
 (segment (start 57.62625 78.105) (end 57.62625 74.295) (width 0.2) (layer "F.Cu") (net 1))
 (segment (start 57.62625 74.295) (end 58.1025 73.81875) (width 0.2) (layer "F.Cu") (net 1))
 (via (at 57.62625 78.105) (size 0.6) (drill 0.3) (layers "F.Cu" "B.Cu") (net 1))
 (segment (start 56.9 78.83125) (end 56.9 81.68875) (width 0.2) (layer "B.Cu") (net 1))
 (segment (start 57.62625 78.105) (end 56.9 78.83125) (width 0.2) (layer "B.Cu") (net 1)))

